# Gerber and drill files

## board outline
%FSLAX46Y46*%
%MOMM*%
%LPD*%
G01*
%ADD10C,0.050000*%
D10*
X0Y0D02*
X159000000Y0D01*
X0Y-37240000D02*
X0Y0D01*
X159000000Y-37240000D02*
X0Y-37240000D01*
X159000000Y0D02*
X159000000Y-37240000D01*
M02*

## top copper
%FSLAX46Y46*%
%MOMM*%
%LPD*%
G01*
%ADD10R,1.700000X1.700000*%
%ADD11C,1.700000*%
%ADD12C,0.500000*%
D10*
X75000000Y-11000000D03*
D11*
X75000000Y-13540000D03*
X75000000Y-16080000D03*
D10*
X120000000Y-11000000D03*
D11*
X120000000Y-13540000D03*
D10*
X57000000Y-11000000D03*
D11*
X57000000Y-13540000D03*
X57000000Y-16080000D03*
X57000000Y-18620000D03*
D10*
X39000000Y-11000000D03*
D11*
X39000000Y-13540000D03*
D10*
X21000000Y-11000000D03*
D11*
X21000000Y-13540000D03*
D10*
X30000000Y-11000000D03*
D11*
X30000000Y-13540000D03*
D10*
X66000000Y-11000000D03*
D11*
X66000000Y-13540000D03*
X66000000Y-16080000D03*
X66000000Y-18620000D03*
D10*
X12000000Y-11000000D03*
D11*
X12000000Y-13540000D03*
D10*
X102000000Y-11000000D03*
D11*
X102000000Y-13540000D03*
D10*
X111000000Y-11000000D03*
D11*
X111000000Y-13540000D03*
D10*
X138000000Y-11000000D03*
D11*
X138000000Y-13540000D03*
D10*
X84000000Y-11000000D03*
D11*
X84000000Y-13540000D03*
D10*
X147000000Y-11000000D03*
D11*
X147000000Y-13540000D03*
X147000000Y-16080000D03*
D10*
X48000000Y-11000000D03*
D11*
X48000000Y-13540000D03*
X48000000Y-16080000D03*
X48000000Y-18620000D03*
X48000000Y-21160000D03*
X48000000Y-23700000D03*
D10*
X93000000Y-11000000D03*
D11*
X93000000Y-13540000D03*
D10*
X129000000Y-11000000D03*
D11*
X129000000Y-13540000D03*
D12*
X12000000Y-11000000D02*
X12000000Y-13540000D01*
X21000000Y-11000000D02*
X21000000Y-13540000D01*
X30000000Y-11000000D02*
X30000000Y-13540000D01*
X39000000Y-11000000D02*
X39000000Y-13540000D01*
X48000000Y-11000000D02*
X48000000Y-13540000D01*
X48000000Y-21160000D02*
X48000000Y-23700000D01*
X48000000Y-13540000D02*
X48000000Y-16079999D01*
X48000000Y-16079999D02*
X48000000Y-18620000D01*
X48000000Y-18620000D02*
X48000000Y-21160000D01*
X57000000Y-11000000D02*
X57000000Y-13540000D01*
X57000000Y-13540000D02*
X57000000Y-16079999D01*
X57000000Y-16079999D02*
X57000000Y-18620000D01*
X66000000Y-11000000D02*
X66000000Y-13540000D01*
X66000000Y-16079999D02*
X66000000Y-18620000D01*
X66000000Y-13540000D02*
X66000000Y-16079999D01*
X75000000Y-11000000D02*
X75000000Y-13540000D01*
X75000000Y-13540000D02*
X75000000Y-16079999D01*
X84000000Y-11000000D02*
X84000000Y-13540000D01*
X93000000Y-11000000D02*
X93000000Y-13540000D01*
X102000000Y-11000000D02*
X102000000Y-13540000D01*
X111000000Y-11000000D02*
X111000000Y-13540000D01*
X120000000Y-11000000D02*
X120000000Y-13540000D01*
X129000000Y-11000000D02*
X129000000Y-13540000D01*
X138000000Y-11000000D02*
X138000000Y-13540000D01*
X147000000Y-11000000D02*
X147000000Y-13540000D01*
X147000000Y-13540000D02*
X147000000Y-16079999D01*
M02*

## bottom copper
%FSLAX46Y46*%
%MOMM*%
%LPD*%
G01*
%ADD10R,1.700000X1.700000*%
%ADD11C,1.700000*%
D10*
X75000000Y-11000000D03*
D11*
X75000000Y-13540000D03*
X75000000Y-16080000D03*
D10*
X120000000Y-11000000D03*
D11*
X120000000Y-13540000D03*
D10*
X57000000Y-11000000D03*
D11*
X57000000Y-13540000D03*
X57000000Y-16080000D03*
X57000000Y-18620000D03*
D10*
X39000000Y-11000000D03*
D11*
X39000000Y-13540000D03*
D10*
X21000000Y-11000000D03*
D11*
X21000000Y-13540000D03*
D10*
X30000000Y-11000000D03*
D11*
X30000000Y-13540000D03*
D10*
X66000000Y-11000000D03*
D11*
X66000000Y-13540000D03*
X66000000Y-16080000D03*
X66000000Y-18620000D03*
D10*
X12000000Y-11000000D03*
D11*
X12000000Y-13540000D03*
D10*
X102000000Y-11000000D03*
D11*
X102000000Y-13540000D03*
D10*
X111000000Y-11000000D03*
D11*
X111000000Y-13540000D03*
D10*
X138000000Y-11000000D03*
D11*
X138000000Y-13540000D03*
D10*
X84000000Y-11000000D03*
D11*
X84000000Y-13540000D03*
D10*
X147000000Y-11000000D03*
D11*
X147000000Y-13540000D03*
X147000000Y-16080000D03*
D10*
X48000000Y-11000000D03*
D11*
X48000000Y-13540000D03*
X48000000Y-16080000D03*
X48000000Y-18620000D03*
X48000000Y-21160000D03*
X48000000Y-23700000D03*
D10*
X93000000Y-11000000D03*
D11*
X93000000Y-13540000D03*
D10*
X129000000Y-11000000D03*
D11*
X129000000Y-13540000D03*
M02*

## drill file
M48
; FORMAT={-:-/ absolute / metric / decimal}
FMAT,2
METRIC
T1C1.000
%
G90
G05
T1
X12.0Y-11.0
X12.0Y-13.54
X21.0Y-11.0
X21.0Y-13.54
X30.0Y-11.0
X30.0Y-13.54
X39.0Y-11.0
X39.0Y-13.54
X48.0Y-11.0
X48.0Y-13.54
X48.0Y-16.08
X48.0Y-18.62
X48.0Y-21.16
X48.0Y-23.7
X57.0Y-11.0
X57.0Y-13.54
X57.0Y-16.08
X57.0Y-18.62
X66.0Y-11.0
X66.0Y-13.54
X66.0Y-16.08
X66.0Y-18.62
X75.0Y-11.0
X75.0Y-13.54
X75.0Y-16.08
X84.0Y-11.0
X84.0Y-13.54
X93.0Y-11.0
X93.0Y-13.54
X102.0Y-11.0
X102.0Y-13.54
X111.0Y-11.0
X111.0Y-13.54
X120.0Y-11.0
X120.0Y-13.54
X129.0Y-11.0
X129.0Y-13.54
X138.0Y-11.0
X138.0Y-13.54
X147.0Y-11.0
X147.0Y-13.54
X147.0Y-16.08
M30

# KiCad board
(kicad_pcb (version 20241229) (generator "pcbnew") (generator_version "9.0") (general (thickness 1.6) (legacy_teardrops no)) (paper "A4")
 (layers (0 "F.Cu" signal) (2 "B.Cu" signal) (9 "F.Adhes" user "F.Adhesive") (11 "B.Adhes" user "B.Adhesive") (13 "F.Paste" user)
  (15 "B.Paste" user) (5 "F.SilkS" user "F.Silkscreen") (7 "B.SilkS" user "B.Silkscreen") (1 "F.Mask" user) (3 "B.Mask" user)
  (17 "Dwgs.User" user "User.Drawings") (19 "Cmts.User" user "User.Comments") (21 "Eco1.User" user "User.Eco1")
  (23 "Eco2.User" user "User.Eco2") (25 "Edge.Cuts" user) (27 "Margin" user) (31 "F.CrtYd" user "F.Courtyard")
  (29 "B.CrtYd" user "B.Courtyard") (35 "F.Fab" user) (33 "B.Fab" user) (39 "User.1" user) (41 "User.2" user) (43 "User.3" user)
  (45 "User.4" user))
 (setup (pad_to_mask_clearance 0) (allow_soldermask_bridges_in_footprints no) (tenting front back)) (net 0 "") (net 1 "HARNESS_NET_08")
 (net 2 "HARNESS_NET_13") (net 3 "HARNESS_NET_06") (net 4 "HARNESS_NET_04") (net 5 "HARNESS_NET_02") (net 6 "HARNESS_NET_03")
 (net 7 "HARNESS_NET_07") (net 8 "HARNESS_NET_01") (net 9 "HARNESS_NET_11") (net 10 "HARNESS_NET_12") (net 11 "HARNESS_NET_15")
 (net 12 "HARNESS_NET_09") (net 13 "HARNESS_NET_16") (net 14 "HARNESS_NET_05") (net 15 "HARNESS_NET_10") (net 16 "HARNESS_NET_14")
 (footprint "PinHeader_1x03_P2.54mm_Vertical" (layer "F.Cu") (at 75 11)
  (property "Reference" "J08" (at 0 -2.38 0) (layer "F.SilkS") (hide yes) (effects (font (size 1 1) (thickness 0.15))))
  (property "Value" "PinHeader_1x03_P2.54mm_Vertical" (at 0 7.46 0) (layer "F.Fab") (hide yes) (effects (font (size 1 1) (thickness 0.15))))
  (pad "1" thru_hole rect (at 0 0) (size 1.7 1.7) (drill 1) (layers "*.Cu" "*.Mask") (remove_unused_layers no) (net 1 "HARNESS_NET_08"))
  (pad "2" thru_hole circle (at 0 2.54) (size 1.7 1.7) (drill 1) (layers "*.Cu" "*.Mask") (remove_unused_layers no) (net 1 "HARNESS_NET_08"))
  (pad "3" thru_hole circle (at 0 5.08) (size 1.7 1.7) (drill 1) (layers "*.Cu" "*.Mask") (remove_unused_layers no) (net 1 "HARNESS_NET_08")))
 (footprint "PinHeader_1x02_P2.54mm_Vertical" (layer "F.Cu") (at 120 11)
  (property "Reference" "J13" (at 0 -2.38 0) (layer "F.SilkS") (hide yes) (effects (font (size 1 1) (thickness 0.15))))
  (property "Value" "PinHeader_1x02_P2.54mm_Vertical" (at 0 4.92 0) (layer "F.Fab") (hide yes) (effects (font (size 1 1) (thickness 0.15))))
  (pad "1" thru_hole rect (at 0 0) (size 1.7 1.7) (drill 1) (layers "*.Cu" "*.Mask") (remove_unused_layers no) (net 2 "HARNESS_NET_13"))
  (pad "2" thru_hole circle (at 0 2.54) (size 1.7 1.7) (drill 1) (layers "*.Cu" "*.Mask") (remove_unused_layers no) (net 2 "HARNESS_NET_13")))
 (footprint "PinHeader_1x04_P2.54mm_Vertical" (layer "F.Cu") (at 57 11)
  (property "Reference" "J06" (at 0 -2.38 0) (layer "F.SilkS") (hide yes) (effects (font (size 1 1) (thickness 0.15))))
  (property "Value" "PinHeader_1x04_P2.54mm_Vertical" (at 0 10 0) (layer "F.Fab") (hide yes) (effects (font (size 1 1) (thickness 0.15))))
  (pad "1" thru_hole rect (at 0 0) (size 1.7 1.7) (drill 1) (layers "*.Cu" "*.Mask") (remove_unused_layers no) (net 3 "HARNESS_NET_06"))
  (pad "2" thru_hole circle (at 0 2.54) (size 1.7 1.7) (drill 1) (layers "*.Cu" "*.Mask") (remove_unused_layers no) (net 3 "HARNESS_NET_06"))
  (pad "3" thru_hole circle (at 0 5.08) (size 1.7 1.7) (drill 1) (layers "*.Cu" "*.Mask") (remove_unused_layers no) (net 3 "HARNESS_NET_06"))
  (pad "4" thru_hole circle (at 0 7.62) (size 1.7 1.7) (drill 1) (layers "*.Cu" "*.Mask") (remove_unused_layers no) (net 3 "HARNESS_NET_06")))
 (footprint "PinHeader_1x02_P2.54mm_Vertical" (layer "F.Cu") (at 39 11)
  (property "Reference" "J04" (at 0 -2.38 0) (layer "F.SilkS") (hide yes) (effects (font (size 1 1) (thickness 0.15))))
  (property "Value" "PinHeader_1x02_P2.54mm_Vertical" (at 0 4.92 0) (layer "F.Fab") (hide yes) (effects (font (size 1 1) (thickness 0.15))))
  (pad "1" thru_hole rect (at 0 0) (size 1.7 1.7) (drill 1) (layers "*.Cu" "*.Mask") (remove_unused_layers no) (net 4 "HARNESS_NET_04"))
  (pad "2" thru_hole circle (at 0 2.54) (size 1.7 1.7) (drill 1) (layers "*.Cu" "*.Mask") (remove_unused_layers no) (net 4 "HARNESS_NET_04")))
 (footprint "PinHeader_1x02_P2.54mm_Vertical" (layer "F.Cu") (at 21 11)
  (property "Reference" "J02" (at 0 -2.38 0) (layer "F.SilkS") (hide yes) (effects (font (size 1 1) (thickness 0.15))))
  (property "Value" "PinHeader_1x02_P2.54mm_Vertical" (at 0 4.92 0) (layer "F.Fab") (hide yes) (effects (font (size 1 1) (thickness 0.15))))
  (pad "1" thru_hole rect (at 0 0) (size 1.7 1.7) (drill 1) (layers "*.Cu" "*.Mask") (remove_unused_layers no) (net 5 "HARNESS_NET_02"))
  (pad "2" thru_hole circle (at 0 2.54) (size 1.7 1.7) (drill 1) (layers "*.Cu" "*.Mask") (remove_unused_layers no) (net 5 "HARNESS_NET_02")))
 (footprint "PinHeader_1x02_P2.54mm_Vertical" (layer "F.Cu") (at 30 11)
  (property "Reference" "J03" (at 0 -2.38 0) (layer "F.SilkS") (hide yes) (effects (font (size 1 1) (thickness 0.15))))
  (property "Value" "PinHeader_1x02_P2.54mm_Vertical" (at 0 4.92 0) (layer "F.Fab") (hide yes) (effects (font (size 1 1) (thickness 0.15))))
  (pad "1" thru_hole rect (at 0 0) (size 1.7 1.7) (drill 1) (layers "*.Cu" "*.Mask") (remove_unused_layers no) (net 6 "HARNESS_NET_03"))
  (pad "2" thru_hole circle (at 0 2.54) (size 1.7 1.7) (drill 1) (layers "*.Cu" "*.Mask") (remove_unused_layers no) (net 6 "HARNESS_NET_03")))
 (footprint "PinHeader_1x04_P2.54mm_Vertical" (layer "F.Cu") (at 66 11)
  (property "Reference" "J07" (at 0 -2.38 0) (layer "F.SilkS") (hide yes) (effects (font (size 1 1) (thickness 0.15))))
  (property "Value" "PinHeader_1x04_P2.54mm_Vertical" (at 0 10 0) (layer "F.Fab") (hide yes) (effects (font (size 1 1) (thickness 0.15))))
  (pad "1" thru_hole rect (at 0 0) (size 1.7 1.7) (drill 1) (layers "*.Cu" "*.Mask") (remove_unused_layers no) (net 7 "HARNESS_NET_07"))
  (pad "2" thru_hole circle (at 0 2.54) (size 1.7 1.7) (drill 1) (layers "*.Cu" "*.Mask") (remove_unused_layers no) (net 7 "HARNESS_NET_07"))
  (pad "3" thru_hole circle (at 0 5.08) (size 1.7 1.7) (drill 1) (layers "*.Cu" "*.Mask") (remove_unused_layers no) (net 7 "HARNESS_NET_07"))
  (pad "4" thru_hole circle (at 0 7.62) (size 1.7 1.7) (drill 1) (layers "*.Cu" "*.Mask") (remove_unused_layers no) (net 7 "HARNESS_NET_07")))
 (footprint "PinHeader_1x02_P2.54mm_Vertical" (layer "F.Cu") (at 12 11)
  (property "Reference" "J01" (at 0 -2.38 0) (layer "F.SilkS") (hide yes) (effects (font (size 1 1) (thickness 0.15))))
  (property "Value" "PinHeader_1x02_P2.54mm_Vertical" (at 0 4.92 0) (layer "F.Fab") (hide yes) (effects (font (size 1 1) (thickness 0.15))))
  (pad "1" thru_hole rect (at 0 0) (size 1.7 1.7) (drill 1) (layers "*.Cu" "*.Mask") (remove_unused_layers no) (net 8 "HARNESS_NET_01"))
  (pad "2" thru_hole circle (at 0 2.54) (size 1.7 1.7) (drill 1) (layers "*.Cu" "*.Mask") (remove_unused_layers no) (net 8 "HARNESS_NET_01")))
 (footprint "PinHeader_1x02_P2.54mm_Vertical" (layer "F.Cu") (at 102 11)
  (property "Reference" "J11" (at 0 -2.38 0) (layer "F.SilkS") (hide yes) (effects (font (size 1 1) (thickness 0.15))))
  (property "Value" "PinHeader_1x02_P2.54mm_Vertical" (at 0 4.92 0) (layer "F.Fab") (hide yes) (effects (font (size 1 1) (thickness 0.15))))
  (pad "1" thru_hole rect (at 0 0) (size 1.7 1.7) (drill 1) (layers "*.Cu" "*.Mask") (remove_unused_layers no) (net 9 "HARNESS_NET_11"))
  (pad "2" thru_hole circle (at 0 2.54) (size 1.7 1.7) (drill 1) (layers "*.Cu" "*.Mask") (remove_unused_layers no) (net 9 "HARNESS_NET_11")))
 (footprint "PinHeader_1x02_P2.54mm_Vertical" (layer "F.Cu") (at 111 11)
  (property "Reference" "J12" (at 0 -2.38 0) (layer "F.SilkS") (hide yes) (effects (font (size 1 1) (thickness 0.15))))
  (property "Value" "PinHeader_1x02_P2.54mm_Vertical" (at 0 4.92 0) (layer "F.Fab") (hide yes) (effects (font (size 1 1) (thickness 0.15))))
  (pad "1" thru_hole rect (at 0 0) (size 1.7 1.7) (drill 1) (layers "*.Cu" "*.Mask") (remove_unused_layers no) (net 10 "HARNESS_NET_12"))
  (pad "2" thru_hole circle (at 0 2.54) (size 1.7 1.7) (drill 1) (layers "*.Cu" "*.Mask") (remove_unused_layers no)
   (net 10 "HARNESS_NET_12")))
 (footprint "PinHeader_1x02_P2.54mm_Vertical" (layer "F.Cu") (at 138 11)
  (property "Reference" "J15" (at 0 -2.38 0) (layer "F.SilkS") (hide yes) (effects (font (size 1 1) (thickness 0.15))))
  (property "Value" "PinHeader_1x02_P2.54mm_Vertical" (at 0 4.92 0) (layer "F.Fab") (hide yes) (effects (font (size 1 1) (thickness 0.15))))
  (pad "1" thru_hole rect (at 0 0) (size 1.7 1.7) (drill 1) (layers "*.Cu" "*.Mask") (remove_unused_layers no) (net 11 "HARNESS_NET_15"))
  (pad "2" thru_hole circle (at 0 2.54) (size 1.7 1.7) (drill 1) (layers "*.Cu" "*.Mask") (remove_unused_layers no)
   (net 11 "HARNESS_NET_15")))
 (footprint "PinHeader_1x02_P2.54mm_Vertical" (layer "F.Cu") (at 84 11)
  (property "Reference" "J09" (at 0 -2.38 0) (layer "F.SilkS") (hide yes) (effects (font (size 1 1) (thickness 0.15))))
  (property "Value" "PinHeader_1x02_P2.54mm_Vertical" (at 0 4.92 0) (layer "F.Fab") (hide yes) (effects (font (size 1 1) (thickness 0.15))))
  (pad "1" thru_hole rect (at 0 0) (size 1.7 1.7) (drill 1) (layers "*.Cu" "*.Mask") (remove_unused_layers no) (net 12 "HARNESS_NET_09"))
  (pad "2" thru_hole circle (at 0 2.54) (size 1.7 1.7) (drill 1) (layers "*.Cu" "*.Mask") (remove_unused_layers no)
   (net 12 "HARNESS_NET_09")))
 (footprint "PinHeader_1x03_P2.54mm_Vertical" (layer "F.Cu") (at 147 11)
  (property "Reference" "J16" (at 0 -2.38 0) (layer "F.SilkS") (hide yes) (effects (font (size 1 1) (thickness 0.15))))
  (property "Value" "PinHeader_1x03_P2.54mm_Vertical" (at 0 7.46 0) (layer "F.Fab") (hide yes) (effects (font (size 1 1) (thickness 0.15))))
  (pad "1" thru_hole rect (at 0 0) (size 1.7 1.7) (drill 1) (layers "*.Cu" "*.Mask") (remove_unused_layers no) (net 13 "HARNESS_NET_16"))
  (pad "2" thru_hole circle (at 0 2.54) (size 1.7 1.7) (drill 1) (layers "*.Cu" "*.Mask") (remove_unused_layers no)
   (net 13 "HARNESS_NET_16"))
  (pad "3" thru_hole circle (at 0 5.08) (size 1.7 1.7) (drill 1) (layers "*.Cu" "*.Mask") (remove_unused_layers no)
   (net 13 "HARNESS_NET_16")))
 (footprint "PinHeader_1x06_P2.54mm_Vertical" (layer "F.Cu") (at 48 11)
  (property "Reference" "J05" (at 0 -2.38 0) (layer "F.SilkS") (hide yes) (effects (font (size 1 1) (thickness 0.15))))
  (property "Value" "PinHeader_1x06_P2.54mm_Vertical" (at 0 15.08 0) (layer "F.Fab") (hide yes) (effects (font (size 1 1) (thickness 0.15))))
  (pad "1" thru_hole rect (at 0 0) (size 1.7 1.7) (drill 1) (layers "*.Cu" "*.Mask") (remove_unused_layers no) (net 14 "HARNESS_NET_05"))
  (pad "2" thru_hole circle (at 0 2.54) (size 1.7 1.7) (drill 1) (layers "*.Cu" "*.Mask") (remove_unused_layers no)
   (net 14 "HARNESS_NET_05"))
  (pad "3" thru_hole circle (at 0 5.08) (size 1.7 1.7) (drill 1) (layers "*.Cu" "*.Mask") (remove_unused_layers no)
   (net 14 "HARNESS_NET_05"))
  (pad "4" thru_hole circle (at 0 7.62) (size 1.7 1.7) (drill 1) (layers "*.Cu" "*.Mask") (remove_unused_layers no)
   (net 14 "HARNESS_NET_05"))
  (pad "5" thru_hole circle (at 0 10.16) (size 1.7 1.7) (drill 1) (layers "*.Cu" "*.Mask") (remove_unused_layers no)
   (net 14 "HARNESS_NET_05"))
  (pad "6" thru_hole circle (at 0 12.7) (size 1.7 1.7) (drill 1) (layers "*.Cu" "*.Mask") (remove_unused_layers no)
   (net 14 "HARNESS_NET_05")))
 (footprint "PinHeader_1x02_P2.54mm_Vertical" (layer "F.Cu") (at 93 11)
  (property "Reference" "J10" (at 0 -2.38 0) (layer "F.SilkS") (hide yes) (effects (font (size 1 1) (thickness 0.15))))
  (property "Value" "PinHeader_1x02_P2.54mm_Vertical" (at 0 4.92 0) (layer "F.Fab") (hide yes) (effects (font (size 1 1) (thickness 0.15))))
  (pad "1" thru_hole rect (at 0 0) (size 1.7 1.7) (drill 1) (layers "*.Cu" "*.Mask") (remove_unused_layers no) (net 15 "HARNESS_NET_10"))
  (pad "2" thru_hole circle (at 0 2.54) (size 1.7 1.7) (drill 1) (layers "*.Cu" "*.Mask") (remove_unused_layers no)
   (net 15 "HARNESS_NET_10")))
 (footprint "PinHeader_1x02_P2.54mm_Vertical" (layer "F.Cu") (at 129 11)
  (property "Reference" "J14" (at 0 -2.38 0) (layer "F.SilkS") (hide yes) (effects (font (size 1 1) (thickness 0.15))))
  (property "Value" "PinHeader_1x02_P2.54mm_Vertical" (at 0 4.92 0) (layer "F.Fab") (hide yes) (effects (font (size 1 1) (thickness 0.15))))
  (pad "1" thru_hole rect (at 0 0) (size 1.7 1.7) (drill 1) (layers "*.Cu" "*.Mask") (remove_unused_layers no) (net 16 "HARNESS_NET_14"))
  (pad "2" thru_hole circle (at 0 2.54) (size 1.7 1.7) (drill 1) (layers "*.Cu" "*.Mask") (remove_unused_layers no)
   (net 16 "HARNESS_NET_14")))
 (gr_line (start 0 0) (end 159 0) (stroke (width 0.05) (type default)) (layer "Edge.Cuts"))
 (gr_line (start 0 37.24) (end 0 0) (stroke (width 0.05) (type default)) (layer "Edge.Cuts"))
 (gr_line (start 159 37.24) (end 0 37.24) (stroke (width 0.05) (type default)) (layer "Edge.Cuts"))
 (gr_line (start 159 0) (end 159 37.24) (stroke (width 0.05) (type default)) (layer "Edge.Cuts"))
 (segment (start 12 11) (end 12 13.54) (width 0.5) (layer "F.Cu") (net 8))
 (segment (start 21 11) (end 21 13.54) (width 0.5) (layer "F.Cu") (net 5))
 (segment (start 30 11) (end 30 13.54) (width 0.5) (layer "F.Cu") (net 6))
 (segment (start 39 11) (end 39 13.54) (width 0.5) (layer "F.Cu") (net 4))
 (segment (start 48 11) (end 48 13.54) (width 0.5) (layer "F.Cu") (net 14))
 (segment (start 48 21.16) (end 48 23.7) (width 0.5) (layer "F.Cu") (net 14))
 (segment (start 48 13.54) (end 48 16.079999) (width 0.5) (layer "F.Cu") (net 14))
 (segment (start 48 16.079999) (end 48 18.62) (width 0.5) (layer "F.Cu") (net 14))
 (segment (start 48 18.62) (end 48 21.16) (width 0.5) (layer "F.Cu") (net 14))
 (segment (start 57 11) (end 57 13.54) (width 0.5) (layer "F.Cu") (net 3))
 (segment (start 57 13.54) (end 57 16.079999) (width 0.5) (layer "F.Cu") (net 3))
 (segment (start 57 16.079999) (end 57 18.62) (width 0.5) (layer "F.Cu") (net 3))
 (segment (start 66 11) (end 66 13.54) (width 0.5) (layer "F.Cu") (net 7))
 (segment (start 66 16.079999) (end 66 18.62) (width 0.5) (layer "F.Cu") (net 7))
 (segment (start 66 13.54) (end 66 16.079999) (width 0.5) (layer "F.Cu") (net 7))
 (segment (start 75 11) (end 75 13.54) (width 0.5) (layer "F.Cu") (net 1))
 (segment (start 75 13.54) (end 75 16.079999) (width 0.5) (layer "F.Cu") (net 1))
 (segment (start 84 11) (end 84 13.54) (width 0.5) (layer "F.Cu") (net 12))
 (segment (start 93 11) (end 93 13.54) (width 0.5) (layer "F.Cu") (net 15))
 (segment (start 102 11) (end 102 13.54) (width 0.5) (layer "F.Cu") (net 9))
 (segment (start 111 11) (end 111 13.54) (width 0.5) (layer "F.Cu") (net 10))
 (segment (start 120 11) (end 120 13.54) (width 0.5) (layer "F.Cu") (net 2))
 (segment (start 129 11) (end 129 13.54) (width 0.5) (layer "F.Cu") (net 16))
 (segment (start 138 11) (end 138 13.54) (width 0.5) (layer "F.Cu") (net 11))
 (segment (start 147 11) (end 147 13.54) (width 0.5) (layer "F.Cu") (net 13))
 (segment (start 147 13.54) (end 147 16.079999) (width 0.5) (layer "F.Cu") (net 13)))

